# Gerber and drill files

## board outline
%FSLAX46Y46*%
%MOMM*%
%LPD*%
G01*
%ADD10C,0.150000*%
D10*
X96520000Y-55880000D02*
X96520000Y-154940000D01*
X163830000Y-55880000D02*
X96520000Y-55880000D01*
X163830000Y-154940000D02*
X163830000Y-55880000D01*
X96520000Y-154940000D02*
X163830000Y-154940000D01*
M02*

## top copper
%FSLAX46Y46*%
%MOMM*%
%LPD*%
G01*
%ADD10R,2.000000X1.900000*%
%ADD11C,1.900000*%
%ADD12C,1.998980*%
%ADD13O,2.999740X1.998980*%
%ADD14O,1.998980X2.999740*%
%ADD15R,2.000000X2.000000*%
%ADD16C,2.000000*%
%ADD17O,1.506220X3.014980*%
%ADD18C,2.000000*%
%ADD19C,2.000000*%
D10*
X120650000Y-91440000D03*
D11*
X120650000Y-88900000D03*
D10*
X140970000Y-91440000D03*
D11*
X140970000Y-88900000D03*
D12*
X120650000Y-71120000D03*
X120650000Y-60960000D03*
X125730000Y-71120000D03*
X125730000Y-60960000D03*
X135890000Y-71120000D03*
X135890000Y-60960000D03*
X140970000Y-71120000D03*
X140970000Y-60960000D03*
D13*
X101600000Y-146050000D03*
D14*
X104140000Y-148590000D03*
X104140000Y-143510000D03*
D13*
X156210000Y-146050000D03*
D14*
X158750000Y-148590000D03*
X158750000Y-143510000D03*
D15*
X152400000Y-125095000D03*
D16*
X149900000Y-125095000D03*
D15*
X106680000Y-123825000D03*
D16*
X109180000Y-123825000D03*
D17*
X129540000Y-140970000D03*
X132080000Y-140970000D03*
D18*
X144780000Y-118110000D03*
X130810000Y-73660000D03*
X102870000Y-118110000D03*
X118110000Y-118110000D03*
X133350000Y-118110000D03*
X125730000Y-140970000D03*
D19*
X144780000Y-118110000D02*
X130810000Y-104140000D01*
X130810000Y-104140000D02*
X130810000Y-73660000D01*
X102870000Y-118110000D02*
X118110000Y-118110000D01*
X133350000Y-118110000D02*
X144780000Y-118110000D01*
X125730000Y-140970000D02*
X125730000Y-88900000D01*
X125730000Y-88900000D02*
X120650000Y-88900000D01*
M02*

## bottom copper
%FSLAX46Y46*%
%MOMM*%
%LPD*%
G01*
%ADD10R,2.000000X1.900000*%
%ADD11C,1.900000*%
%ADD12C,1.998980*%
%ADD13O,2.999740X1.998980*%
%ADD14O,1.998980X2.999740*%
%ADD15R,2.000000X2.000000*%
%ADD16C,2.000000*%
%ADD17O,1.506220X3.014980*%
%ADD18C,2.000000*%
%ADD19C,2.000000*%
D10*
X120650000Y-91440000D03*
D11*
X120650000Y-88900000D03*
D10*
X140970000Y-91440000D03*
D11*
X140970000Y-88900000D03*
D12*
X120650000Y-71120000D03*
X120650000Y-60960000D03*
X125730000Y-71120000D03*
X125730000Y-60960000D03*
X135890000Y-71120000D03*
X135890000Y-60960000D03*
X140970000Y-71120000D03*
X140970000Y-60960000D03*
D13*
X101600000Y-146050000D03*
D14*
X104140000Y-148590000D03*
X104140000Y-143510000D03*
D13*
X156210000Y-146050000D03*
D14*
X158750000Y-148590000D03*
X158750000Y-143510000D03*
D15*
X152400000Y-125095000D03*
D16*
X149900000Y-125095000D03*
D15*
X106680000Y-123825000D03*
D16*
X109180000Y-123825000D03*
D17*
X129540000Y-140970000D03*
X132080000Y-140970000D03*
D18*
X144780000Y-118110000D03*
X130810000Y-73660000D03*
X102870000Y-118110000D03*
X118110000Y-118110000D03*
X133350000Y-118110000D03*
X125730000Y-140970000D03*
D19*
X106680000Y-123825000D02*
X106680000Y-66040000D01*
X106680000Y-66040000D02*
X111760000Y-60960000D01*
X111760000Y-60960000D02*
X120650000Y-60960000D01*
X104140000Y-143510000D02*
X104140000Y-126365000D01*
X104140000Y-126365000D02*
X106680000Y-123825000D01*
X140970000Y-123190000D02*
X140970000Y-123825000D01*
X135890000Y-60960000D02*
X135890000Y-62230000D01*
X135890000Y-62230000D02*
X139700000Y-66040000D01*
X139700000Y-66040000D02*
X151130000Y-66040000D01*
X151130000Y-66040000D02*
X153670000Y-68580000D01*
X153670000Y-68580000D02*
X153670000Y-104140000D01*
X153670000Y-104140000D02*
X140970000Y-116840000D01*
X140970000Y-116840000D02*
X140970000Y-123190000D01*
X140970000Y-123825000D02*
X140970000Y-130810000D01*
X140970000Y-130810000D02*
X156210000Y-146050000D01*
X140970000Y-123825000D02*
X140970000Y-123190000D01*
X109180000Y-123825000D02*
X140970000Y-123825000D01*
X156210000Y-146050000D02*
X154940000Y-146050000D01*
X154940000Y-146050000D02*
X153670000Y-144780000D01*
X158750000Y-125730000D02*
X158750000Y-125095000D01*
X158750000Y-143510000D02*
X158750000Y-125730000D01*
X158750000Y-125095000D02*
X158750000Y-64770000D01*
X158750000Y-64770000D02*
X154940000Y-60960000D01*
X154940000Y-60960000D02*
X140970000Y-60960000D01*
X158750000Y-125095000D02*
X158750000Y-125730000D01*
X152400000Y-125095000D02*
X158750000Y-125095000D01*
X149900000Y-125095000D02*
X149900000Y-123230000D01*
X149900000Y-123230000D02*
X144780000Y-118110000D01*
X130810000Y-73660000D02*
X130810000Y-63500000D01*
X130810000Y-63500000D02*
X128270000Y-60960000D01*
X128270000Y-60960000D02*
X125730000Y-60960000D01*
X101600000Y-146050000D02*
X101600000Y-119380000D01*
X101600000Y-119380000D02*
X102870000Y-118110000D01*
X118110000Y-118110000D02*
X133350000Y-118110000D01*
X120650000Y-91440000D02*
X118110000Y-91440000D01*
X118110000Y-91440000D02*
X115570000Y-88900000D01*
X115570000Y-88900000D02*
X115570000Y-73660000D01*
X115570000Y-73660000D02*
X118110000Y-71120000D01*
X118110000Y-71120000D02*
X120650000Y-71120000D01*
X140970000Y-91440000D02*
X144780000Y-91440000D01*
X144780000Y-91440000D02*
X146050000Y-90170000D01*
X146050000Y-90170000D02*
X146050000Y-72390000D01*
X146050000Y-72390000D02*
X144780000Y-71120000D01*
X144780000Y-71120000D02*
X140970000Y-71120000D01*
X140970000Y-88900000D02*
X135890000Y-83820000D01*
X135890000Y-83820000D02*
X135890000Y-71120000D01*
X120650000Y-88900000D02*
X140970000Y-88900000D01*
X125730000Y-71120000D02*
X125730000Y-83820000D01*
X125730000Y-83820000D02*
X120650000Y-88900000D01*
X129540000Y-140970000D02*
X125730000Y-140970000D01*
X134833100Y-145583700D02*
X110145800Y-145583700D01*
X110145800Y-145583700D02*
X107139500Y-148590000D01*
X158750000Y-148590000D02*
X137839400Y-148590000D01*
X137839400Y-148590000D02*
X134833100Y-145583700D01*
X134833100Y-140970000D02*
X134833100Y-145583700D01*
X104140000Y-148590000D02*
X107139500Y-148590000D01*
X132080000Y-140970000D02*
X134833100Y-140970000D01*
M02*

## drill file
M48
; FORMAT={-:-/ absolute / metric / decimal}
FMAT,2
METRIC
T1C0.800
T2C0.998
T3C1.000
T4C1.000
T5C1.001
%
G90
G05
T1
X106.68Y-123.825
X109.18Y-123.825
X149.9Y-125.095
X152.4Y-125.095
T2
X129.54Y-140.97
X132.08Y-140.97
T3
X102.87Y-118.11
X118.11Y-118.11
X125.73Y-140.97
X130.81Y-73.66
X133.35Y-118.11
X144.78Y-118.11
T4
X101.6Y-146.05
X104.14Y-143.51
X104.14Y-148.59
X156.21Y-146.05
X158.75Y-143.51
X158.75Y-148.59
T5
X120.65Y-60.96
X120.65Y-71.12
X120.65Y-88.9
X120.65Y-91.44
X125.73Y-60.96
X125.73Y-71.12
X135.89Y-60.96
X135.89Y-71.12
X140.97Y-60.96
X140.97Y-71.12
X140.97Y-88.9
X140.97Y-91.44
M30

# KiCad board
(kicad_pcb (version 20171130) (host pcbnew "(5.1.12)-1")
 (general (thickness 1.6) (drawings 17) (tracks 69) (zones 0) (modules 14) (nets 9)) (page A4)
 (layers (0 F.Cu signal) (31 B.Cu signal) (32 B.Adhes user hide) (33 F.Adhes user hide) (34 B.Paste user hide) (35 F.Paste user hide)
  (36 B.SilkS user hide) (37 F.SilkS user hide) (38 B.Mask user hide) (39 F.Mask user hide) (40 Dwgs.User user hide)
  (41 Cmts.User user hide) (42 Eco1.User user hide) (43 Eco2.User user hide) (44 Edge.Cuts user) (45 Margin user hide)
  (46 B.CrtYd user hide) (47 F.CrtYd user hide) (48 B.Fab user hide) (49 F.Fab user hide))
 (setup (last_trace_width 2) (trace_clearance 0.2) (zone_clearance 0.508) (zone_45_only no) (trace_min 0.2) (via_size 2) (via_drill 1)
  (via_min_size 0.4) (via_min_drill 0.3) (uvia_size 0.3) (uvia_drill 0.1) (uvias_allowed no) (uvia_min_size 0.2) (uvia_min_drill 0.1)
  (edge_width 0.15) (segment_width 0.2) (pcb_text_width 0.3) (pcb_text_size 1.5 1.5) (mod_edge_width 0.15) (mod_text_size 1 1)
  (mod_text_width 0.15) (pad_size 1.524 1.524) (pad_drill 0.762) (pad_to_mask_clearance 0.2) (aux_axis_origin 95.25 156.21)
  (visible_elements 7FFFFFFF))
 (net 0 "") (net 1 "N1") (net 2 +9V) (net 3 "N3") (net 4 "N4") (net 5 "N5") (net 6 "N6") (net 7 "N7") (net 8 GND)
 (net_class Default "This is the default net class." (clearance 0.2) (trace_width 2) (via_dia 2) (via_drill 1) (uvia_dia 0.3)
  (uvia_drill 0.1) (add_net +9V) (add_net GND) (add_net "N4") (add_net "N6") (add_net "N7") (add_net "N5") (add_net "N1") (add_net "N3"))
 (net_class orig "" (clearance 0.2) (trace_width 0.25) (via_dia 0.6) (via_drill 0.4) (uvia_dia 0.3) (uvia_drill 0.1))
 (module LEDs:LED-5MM (layer F.Cu) (at 120.65 91.44 90)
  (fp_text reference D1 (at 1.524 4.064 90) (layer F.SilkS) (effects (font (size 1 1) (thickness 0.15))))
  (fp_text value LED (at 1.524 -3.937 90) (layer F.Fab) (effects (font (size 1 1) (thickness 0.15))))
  (pad 1 thru_hole rect (at 0 0 180) (size 2 1.9) (drill 1.00076) (layers *.Cu *.Mask) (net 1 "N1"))
  (pad 2 thru_hole circle (at 2.54 0 90) (size 1.9 1.9) (drill 1.00076) (layers *.Cu *.Mask) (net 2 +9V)))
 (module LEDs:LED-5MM (layer F.Cu) (at 140.97 91.44 90)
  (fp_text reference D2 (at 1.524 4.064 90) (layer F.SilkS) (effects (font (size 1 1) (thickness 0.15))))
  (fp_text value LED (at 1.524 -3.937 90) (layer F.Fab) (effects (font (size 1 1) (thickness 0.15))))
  (pad 1 thru_hole rect (at 0 0 180) (size 2 1.9) (drill 1.00076) (layers *.Cu *.Mask) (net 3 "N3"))
  (pad 2 thru_hole circle (at 2.54 0 90) (size 1.9 1.9) (drill 1.00076) (layers *.Cu *.Mask) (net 2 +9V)))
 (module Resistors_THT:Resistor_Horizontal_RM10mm (layer F.Cu) (at 120.65 71.12 90)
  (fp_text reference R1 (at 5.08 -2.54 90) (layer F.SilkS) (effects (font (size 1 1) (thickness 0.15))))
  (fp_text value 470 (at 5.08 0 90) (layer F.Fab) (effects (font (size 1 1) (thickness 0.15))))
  (pad 1 thru_hole circle (at 0 0 90) (size 1.99898 1.99898) (drill 1.00076) (layers *.Cu *.SilkS *.Mask) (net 1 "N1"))
  (pad 2 thru_hole circle (at 10.16 0 90) (size 1.99898 1.99898) (drill 1.00076) (layers *.Cu *.SilkS *.Mask) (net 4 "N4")))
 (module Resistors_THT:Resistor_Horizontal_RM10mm (layer F.Cu) (at 125.73 71.12 90)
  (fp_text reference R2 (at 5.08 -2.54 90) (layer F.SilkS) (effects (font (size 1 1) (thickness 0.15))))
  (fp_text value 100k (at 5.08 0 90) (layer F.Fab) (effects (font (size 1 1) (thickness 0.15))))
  (pad 1 thru_hole circle (at 0 0 90) (size 1.99898 1.99898) (drill 1.00076) (layers *.Cu *.SilkS *.Mask) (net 2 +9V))
  (pad 2 thru_hole circle (at 10.16 0 90) (size 1.99898 1.99898) (drill 1.00076) (layers *.Cu *.SilkS *.Mask) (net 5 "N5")))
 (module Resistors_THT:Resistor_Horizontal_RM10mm (layer F.Cu) (at 135.89 71.12 90)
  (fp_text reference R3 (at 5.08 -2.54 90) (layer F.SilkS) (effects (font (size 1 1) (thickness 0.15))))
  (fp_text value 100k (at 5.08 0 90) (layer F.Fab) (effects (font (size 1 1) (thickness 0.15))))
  (pad 1 thru_hole circle (at 0 0 90) (size 1.99898 1.99898) (drill 1.00076) (layers *.Cu *.SilkS *.Mask) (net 2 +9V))
  (pad 2 thru_hole circle (at 10.16 0 90) (size 1.99898 1.99898) (drill 1.00076) (layers *.Cu *.SilkS *.Mask) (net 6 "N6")))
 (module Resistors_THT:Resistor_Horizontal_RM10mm (layer F.Cu) (at 140.97 71.12 90)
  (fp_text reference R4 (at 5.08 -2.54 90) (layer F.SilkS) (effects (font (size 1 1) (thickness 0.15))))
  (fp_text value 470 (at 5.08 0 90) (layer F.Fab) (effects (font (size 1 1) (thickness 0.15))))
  (pad 1 thru_hole circle (at 0 0 90) (size 1.99898 1.99898) (drill 1.00076) (layers *.Cu *.SilkS *.Mask) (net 3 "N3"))
  (pad 2 thru_hole circle (at 10.16 0 90) (size 1.99898 1.99898) (drill 1.00076) (layers *.Cu *.SilkS *.Mask) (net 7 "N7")))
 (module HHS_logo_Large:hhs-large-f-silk (layer F.Cu) (at 130.81 103.505)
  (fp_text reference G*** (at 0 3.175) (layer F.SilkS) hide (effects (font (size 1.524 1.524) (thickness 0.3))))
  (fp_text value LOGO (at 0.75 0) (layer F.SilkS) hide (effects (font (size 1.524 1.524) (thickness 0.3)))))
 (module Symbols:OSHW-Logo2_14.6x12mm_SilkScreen (layer B.Cu) (at 139.7 109.22 180)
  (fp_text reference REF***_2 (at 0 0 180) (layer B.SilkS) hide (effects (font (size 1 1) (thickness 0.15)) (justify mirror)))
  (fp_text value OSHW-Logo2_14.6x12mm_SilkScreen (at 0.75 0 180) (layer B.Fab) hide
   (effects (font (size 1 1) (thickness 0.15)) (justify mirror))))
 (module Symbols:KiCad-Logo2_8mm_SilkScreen (layer B.Cu) (at 118.11 110.49 180)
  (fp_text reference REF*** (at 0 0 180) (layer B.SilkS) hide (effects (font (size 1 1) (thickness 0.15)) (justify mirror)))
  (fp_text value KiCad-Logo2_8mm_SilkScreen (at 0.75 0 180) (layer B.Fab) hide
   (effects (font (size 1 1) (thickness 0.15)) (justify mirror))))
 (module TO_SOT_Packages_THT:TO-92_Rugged (layer F.Cu) (at 104.14 148.59 90)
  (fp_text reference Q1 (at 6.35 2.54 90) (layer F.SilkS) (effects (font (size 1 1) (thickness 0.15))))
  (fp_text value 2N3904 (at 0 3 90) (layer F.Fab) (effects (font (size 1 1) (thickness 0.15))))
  (pad 2 thru_hole oval (at 2.54 -2.54 180) (size 2.99974 1.99898) (drill 1) (layers *.Cu *.Mask) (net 5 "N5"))
  (pad 1 thru_hole oval (at 0 0 180) (size 1.99898 2.99974) (drill 1) (layers *.Cu *.Mask) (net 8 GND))
  (pad 3 thru_hole oval (at 5.08 0 180) (size 1.99898 2.99974) (drill 1) (layers *.Cu *.Mask) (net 4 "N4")))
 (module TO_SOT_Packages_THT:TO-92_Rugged (layer F.Cu) (at 158.75 148.59 90)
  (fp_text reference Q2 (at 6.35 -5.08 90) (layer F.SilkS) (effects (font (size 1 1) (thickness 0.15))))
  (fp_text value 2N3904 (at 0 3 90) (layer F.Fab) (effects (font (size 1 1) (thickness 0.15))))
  (pad 2 thru_hole oval (at 2.54 -2.54 180) (size 2.99974 1.99898) (drill 1) (layers *.Cu *.Mask) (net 6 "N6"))
  (pad 1 thru_hole oval (at 0 0 180) (size 1.99898 2.99974) (drill 1) (layers *.Cu *.Mask) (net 8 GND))
  (pad 3 thru_hole oval (at 5.08 0 180) (size 1.99898 2.99974) (drill 1) (layers *.Cu *.Mask) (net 7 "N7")))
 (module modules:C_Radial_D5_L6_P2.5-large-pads (layer F.Cu) (at 152.4 125.095 180)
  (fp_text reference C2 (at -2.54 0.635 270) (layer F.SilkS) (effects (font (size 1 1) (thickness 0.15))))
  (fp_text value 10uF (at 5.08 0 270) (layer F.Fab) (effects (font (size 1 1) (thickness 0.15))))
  (pad 1 thru_hole rect (at 0 0 180) (size 2 2) (drill 0.8) (layers *.Cu *.Mask) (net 7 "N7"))
  (pad 2 thru_hole circle (at 2.5 0 180) (size 2 2) (drill 0.8) (layers *.Cu *.Mask) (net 5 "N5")))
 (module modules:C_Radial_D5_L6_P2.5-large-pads (layer F.Cu) (at 106.68 123.825)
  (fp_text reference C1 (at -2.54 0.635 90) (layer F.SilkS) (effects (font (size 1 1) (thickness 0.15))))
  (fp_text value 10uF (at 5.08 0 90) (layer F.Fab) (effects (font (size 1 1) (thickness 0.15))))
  (pad 1 thru_hole rect (at 0 0) (size 2 2) (drill 0.8) (layers *.Cu *.Mask) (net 4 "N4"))
  (pad 2 thru_hole circle (at 2.5 0) (size 2 2) (drill 0.8) (layers *.Cu *.Mask) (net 6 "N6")))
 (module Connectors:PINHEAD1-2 (layer B.Cu) (at 130.81 140.97)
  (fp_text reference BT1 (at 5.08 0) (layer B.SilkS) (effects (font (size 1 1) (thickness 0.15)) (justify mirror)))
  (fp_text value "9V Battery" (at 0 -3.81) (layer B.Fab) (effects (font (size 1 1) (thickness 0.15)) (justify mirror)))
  (pad 1 thru_hole oval (at -1.27 0) (size 1.50622 3.01498) (drill 0.99822) (layers *.Cu *.Mask) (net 2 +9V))
  (pad 2 thru_hole oval (at 1.27 0) (size 1.50622 3.01498) (drill 0.99822) (layers *.Cu *.Mask) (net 8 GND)))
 (gr_line (start 96.52 55.88) (end 96.52 154.94) (angle 90) (layer Edge.Cuts) (width 0.15))
 (gr_line (start 163.83 55.88) (end 96.52 55.88) (angle 90) (layer Edge.Cuts) (width 0.15))
 (gr_line (start 163.83 154.94) (end 163.83 55.88) (angle 90) (layer Edge.Cuts) (width 0.15))
 (gr_line (start 96.52 154.94) (end 163.83 154.94) (angle 90) (layer Edge.Cuts) (width 0.15))
 (segment (start 106.68 123.825) (end 106.68 66.04) (width 2) (layer B.Cu) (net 4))
 (segment (start 106.68 66.04) (end 111.76 60.96) (width 2) (layer B.Cu) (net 4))
 (segment (start 111.76 60.96) (end 120.65 60.96) (width 2) (layer B.Cu) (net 4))
 (segment (start 104.14 143.51) (end 104.14 126.365) (width 2) (layer B.Cu) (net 4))
 (segment (start 104.14 126.365) (end 106.68 123.825) (width 2) (layer B.Cu) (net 4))
 (segment (start 140.97 123.19) (end 140.97 123.825) (width 2) (layer B.Cu) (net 6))
 (segment (start 135.89 60.96) (end 135.89 62.23) (width 2) (layer B.Cu) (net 6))
 (segment (start 135.89 62.23) (end 139.7 66.04) (width 2) (layer B.Cu) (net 6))
 (segment (start 139.7 66.04) (end 151.13 66.04) (width 2) (layer B.Cu) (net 6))
 (segment (start 151.13 66.04) (end 153.67 68.58) (width 2) (layer B.Cu) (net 6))
 (segment (start 153.67 68.58) (end 153.67 104.14) (width 2) (layer B.Cu) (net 6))
 (segment (start 153.67 104.14) (end 140.97 116.84) (width 2) (layer B.Cu) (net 6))
 (segment (start 140.97 116.84) (end 140.97 123.19) (width 2) (layer B.Cu) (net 6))
 (segment (start 140.97 123.825) (end 140.97 130.81) (width 2) (layer B.Cu) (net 6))
 (segment (start 140.97 130.81) (end 156.21 146.05) (width 2) (layer B.Cu) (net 6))
 (segment (start 140.97 123.825) (end 140.97 123.19) (width 2) (layer B.Cu) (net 6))
 (segment (start 109.18 123.825) (end 140.97 123.825) (width 2) (layer B.Cu) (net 6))
 (segment (start 156.21 146.05) (end 154.94 146.05) (width 2) (layer B.Cu) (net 6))
 (segment (start 154.94 146.05) (end 153.67 144.78) (width 2) (layer B.Cu) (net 6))
 (segment (start 158.75 125.73) (end 158.75 125.095) (width 2) (layer B.Cu) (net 7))
 (segment (start 158.75 143.51) (end 158.75 125.73) (width 2) (layer B.Cu) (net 7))
 (segment (start 158.75 125.095) (end 158.75 64.77) (width 2) (layer B.Cu) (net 7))
 (segment (start 158.75 64.77) (end 154.94 60.96) (width 2) (layer B.Cu) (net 7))
 (segment (start 154.94 60.96) (end 140.97 60.96) (width 2) (layer B.Cu) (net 7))
 (segment (start 158.75 125.095) (end 158.75 125.73) (width 2) (layer B.Cu) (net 7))
 (segment (start 152.4 125.095) (end 158.75 125.095) (width 2) (layer B.Cu) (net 7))
 (segment (start 149.9 125.095) (end 149.9 123.23) (width 2) (layer B.Cu) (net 5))
 (segment (start 149.9 123.23) (end 144.78 118.11) (width 2) (layer B.Cu) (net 5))
 (segment (start 144.78 118.11) (end 130.81 104.14) (width 2) (layer F.Cu) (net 5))
 (segment (start 130.81 104.14) (end 130.81 73.66) (width 2) (layer F.Cu) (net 5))
 (segment (start 130.81 73.66) (end 130.81 63.5) (width 2) (layer B.Cu) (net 5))
 (segment (start 130.81 63.5) (end 128.27 60.96) (width 2) (layer B.Cu) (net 5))
 (segment (start 128.27 60.96) (end 125.73 60.96) (width 2) (layer B.Cu) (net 5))
 (segment (start 101.6 146.05) (end 101.6 119.38) (width 2) (layer B.Cu) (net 5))
 (segment (start 101.6 119.38) (end 102.87 118.11) (width 2) (layer B.Cu) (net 5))
 (segment (start 102.87 118.11) (end 118.11 118.11) (width 2) (layer F.Cu) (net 5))
 (segment (start 118.11 118.11) (end 133.35 118.11) (width 2) (layer B.Cu) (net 5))
 (segment (start 133.35 118.11) (end 144.78 118.11) (width 2) (layer F.Cu) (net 5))
 (via (at 144.78 118.11) (size 2) (layers F.Cu B.Cu) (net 5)) (via (at 130.81 73.66) (size 2) (layers F.Cu B.Cu) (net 5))
 (via (at 102.87 118.11) (size 2) (layers F.Cu B.Cu) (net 5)) (via (at 118.11 118.11) (size 2) (layers F.Cu B.Cu) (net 5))
 (via (at 133.35 118.11) (size 2) (layers F.Cu B.Cu) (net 5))
 (segment (start 120.65 91.44) (end 118.11 91.44) (width 2) (layer B.Cu) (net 1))
 (segment (start 118.11 91.44) (end 115.57 88.9) (width 2) (layer B.Cu) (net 1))
 (segment (start 115.57 88.9) (end 115.57 73.66) (width 2) (layer B.Cu) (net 1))
 (segment (start 115.57 73.66) (end 118.11 71.12) (width 2) (layer B.Cu) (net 1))
 (segment (start 118.11 71.12) (end 120.65 71.12) (width 2) (layer B.Cu) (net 1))
 (segment (start 140.97 91.44) (end 144.78 91.44) (width 2) (layer B.Cu) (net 3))
 (segment (start 144.78 91.44) (end 146.05 90.17) (width 2) (layer B.Cu) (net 3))
 (segment (start 146.05 90.17) (end 146.05 72.39) (width 2) (layer B.Cu) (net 3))
 (segment (start 146.05 72.39) (end 144.78 71.12) (width 2) (layer B.Cu) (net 3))
 (segment (start 144.78 71.12) (end 140.97 71.12) (width 2) (layer B.Cu) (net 3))
 (segment (start 140.97 88.9) (end 135.89 83.82) (width 2) (layer B.Cu) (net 2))
 (segment (start 135.89 83.82) (end 135.89 71.12) (width 2) (layer B.Cu) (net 2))
 (segment (start 120.65 88.9) (end 140.97 88.9) (width 2) (layer B.Cu) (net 2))
 (segment (start 125.73 71.12) (end 125.73 83.82) (width 2) (layer B.Cu) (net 2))
 (segment (start 125.73 83.82) (end 120.65 88.9) (width 2) (layer B.Cu) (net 2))
 (segment (start 125.73 140.97) (end 125.73 88.9) (width 2) (layer F.Cu) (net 2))
 (segment (start 125.73 88.9) (end 120.65 88.9) (width 2) (layer F.Cu) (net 2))
 (segment (start 129.54 140.97) (end 125.73 140.97) (width 2) (layer B.Cu) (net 2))
 (via (at 125.73 140.97) (size 2) (layers F.Cu B.Cu) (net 2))
 (segment (start 134.8331 145.5837) (end 110.1458 145.5837) (width 2) (layer B.Cu) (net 8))
 (segment (start 110.1458 145.5837) (end 107.1395 148.59) (width 2) (layer B.Cu) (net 8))
 (segment (start 158.75 148.59) (end 137.8394 148.59) (width 2) (layer B.Cu) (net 8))
 (segment (start 137.8394 148.59) (end 134.8331 145.5837) (width 2) (layer B.Cu) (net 8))
 (segment (start 134.8331 140.97) (end 134.8331 145.5837) (width 2) (layer B.Cu) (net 8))
 (segment (start 104.14 148.59) (end 107.1395 148.59) (width 2) (layer B.Cu) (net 8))
 (segment (start 132.08 140.97) (end 134.8331 140.97) (width 2) (layer B.Cu) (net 8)))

